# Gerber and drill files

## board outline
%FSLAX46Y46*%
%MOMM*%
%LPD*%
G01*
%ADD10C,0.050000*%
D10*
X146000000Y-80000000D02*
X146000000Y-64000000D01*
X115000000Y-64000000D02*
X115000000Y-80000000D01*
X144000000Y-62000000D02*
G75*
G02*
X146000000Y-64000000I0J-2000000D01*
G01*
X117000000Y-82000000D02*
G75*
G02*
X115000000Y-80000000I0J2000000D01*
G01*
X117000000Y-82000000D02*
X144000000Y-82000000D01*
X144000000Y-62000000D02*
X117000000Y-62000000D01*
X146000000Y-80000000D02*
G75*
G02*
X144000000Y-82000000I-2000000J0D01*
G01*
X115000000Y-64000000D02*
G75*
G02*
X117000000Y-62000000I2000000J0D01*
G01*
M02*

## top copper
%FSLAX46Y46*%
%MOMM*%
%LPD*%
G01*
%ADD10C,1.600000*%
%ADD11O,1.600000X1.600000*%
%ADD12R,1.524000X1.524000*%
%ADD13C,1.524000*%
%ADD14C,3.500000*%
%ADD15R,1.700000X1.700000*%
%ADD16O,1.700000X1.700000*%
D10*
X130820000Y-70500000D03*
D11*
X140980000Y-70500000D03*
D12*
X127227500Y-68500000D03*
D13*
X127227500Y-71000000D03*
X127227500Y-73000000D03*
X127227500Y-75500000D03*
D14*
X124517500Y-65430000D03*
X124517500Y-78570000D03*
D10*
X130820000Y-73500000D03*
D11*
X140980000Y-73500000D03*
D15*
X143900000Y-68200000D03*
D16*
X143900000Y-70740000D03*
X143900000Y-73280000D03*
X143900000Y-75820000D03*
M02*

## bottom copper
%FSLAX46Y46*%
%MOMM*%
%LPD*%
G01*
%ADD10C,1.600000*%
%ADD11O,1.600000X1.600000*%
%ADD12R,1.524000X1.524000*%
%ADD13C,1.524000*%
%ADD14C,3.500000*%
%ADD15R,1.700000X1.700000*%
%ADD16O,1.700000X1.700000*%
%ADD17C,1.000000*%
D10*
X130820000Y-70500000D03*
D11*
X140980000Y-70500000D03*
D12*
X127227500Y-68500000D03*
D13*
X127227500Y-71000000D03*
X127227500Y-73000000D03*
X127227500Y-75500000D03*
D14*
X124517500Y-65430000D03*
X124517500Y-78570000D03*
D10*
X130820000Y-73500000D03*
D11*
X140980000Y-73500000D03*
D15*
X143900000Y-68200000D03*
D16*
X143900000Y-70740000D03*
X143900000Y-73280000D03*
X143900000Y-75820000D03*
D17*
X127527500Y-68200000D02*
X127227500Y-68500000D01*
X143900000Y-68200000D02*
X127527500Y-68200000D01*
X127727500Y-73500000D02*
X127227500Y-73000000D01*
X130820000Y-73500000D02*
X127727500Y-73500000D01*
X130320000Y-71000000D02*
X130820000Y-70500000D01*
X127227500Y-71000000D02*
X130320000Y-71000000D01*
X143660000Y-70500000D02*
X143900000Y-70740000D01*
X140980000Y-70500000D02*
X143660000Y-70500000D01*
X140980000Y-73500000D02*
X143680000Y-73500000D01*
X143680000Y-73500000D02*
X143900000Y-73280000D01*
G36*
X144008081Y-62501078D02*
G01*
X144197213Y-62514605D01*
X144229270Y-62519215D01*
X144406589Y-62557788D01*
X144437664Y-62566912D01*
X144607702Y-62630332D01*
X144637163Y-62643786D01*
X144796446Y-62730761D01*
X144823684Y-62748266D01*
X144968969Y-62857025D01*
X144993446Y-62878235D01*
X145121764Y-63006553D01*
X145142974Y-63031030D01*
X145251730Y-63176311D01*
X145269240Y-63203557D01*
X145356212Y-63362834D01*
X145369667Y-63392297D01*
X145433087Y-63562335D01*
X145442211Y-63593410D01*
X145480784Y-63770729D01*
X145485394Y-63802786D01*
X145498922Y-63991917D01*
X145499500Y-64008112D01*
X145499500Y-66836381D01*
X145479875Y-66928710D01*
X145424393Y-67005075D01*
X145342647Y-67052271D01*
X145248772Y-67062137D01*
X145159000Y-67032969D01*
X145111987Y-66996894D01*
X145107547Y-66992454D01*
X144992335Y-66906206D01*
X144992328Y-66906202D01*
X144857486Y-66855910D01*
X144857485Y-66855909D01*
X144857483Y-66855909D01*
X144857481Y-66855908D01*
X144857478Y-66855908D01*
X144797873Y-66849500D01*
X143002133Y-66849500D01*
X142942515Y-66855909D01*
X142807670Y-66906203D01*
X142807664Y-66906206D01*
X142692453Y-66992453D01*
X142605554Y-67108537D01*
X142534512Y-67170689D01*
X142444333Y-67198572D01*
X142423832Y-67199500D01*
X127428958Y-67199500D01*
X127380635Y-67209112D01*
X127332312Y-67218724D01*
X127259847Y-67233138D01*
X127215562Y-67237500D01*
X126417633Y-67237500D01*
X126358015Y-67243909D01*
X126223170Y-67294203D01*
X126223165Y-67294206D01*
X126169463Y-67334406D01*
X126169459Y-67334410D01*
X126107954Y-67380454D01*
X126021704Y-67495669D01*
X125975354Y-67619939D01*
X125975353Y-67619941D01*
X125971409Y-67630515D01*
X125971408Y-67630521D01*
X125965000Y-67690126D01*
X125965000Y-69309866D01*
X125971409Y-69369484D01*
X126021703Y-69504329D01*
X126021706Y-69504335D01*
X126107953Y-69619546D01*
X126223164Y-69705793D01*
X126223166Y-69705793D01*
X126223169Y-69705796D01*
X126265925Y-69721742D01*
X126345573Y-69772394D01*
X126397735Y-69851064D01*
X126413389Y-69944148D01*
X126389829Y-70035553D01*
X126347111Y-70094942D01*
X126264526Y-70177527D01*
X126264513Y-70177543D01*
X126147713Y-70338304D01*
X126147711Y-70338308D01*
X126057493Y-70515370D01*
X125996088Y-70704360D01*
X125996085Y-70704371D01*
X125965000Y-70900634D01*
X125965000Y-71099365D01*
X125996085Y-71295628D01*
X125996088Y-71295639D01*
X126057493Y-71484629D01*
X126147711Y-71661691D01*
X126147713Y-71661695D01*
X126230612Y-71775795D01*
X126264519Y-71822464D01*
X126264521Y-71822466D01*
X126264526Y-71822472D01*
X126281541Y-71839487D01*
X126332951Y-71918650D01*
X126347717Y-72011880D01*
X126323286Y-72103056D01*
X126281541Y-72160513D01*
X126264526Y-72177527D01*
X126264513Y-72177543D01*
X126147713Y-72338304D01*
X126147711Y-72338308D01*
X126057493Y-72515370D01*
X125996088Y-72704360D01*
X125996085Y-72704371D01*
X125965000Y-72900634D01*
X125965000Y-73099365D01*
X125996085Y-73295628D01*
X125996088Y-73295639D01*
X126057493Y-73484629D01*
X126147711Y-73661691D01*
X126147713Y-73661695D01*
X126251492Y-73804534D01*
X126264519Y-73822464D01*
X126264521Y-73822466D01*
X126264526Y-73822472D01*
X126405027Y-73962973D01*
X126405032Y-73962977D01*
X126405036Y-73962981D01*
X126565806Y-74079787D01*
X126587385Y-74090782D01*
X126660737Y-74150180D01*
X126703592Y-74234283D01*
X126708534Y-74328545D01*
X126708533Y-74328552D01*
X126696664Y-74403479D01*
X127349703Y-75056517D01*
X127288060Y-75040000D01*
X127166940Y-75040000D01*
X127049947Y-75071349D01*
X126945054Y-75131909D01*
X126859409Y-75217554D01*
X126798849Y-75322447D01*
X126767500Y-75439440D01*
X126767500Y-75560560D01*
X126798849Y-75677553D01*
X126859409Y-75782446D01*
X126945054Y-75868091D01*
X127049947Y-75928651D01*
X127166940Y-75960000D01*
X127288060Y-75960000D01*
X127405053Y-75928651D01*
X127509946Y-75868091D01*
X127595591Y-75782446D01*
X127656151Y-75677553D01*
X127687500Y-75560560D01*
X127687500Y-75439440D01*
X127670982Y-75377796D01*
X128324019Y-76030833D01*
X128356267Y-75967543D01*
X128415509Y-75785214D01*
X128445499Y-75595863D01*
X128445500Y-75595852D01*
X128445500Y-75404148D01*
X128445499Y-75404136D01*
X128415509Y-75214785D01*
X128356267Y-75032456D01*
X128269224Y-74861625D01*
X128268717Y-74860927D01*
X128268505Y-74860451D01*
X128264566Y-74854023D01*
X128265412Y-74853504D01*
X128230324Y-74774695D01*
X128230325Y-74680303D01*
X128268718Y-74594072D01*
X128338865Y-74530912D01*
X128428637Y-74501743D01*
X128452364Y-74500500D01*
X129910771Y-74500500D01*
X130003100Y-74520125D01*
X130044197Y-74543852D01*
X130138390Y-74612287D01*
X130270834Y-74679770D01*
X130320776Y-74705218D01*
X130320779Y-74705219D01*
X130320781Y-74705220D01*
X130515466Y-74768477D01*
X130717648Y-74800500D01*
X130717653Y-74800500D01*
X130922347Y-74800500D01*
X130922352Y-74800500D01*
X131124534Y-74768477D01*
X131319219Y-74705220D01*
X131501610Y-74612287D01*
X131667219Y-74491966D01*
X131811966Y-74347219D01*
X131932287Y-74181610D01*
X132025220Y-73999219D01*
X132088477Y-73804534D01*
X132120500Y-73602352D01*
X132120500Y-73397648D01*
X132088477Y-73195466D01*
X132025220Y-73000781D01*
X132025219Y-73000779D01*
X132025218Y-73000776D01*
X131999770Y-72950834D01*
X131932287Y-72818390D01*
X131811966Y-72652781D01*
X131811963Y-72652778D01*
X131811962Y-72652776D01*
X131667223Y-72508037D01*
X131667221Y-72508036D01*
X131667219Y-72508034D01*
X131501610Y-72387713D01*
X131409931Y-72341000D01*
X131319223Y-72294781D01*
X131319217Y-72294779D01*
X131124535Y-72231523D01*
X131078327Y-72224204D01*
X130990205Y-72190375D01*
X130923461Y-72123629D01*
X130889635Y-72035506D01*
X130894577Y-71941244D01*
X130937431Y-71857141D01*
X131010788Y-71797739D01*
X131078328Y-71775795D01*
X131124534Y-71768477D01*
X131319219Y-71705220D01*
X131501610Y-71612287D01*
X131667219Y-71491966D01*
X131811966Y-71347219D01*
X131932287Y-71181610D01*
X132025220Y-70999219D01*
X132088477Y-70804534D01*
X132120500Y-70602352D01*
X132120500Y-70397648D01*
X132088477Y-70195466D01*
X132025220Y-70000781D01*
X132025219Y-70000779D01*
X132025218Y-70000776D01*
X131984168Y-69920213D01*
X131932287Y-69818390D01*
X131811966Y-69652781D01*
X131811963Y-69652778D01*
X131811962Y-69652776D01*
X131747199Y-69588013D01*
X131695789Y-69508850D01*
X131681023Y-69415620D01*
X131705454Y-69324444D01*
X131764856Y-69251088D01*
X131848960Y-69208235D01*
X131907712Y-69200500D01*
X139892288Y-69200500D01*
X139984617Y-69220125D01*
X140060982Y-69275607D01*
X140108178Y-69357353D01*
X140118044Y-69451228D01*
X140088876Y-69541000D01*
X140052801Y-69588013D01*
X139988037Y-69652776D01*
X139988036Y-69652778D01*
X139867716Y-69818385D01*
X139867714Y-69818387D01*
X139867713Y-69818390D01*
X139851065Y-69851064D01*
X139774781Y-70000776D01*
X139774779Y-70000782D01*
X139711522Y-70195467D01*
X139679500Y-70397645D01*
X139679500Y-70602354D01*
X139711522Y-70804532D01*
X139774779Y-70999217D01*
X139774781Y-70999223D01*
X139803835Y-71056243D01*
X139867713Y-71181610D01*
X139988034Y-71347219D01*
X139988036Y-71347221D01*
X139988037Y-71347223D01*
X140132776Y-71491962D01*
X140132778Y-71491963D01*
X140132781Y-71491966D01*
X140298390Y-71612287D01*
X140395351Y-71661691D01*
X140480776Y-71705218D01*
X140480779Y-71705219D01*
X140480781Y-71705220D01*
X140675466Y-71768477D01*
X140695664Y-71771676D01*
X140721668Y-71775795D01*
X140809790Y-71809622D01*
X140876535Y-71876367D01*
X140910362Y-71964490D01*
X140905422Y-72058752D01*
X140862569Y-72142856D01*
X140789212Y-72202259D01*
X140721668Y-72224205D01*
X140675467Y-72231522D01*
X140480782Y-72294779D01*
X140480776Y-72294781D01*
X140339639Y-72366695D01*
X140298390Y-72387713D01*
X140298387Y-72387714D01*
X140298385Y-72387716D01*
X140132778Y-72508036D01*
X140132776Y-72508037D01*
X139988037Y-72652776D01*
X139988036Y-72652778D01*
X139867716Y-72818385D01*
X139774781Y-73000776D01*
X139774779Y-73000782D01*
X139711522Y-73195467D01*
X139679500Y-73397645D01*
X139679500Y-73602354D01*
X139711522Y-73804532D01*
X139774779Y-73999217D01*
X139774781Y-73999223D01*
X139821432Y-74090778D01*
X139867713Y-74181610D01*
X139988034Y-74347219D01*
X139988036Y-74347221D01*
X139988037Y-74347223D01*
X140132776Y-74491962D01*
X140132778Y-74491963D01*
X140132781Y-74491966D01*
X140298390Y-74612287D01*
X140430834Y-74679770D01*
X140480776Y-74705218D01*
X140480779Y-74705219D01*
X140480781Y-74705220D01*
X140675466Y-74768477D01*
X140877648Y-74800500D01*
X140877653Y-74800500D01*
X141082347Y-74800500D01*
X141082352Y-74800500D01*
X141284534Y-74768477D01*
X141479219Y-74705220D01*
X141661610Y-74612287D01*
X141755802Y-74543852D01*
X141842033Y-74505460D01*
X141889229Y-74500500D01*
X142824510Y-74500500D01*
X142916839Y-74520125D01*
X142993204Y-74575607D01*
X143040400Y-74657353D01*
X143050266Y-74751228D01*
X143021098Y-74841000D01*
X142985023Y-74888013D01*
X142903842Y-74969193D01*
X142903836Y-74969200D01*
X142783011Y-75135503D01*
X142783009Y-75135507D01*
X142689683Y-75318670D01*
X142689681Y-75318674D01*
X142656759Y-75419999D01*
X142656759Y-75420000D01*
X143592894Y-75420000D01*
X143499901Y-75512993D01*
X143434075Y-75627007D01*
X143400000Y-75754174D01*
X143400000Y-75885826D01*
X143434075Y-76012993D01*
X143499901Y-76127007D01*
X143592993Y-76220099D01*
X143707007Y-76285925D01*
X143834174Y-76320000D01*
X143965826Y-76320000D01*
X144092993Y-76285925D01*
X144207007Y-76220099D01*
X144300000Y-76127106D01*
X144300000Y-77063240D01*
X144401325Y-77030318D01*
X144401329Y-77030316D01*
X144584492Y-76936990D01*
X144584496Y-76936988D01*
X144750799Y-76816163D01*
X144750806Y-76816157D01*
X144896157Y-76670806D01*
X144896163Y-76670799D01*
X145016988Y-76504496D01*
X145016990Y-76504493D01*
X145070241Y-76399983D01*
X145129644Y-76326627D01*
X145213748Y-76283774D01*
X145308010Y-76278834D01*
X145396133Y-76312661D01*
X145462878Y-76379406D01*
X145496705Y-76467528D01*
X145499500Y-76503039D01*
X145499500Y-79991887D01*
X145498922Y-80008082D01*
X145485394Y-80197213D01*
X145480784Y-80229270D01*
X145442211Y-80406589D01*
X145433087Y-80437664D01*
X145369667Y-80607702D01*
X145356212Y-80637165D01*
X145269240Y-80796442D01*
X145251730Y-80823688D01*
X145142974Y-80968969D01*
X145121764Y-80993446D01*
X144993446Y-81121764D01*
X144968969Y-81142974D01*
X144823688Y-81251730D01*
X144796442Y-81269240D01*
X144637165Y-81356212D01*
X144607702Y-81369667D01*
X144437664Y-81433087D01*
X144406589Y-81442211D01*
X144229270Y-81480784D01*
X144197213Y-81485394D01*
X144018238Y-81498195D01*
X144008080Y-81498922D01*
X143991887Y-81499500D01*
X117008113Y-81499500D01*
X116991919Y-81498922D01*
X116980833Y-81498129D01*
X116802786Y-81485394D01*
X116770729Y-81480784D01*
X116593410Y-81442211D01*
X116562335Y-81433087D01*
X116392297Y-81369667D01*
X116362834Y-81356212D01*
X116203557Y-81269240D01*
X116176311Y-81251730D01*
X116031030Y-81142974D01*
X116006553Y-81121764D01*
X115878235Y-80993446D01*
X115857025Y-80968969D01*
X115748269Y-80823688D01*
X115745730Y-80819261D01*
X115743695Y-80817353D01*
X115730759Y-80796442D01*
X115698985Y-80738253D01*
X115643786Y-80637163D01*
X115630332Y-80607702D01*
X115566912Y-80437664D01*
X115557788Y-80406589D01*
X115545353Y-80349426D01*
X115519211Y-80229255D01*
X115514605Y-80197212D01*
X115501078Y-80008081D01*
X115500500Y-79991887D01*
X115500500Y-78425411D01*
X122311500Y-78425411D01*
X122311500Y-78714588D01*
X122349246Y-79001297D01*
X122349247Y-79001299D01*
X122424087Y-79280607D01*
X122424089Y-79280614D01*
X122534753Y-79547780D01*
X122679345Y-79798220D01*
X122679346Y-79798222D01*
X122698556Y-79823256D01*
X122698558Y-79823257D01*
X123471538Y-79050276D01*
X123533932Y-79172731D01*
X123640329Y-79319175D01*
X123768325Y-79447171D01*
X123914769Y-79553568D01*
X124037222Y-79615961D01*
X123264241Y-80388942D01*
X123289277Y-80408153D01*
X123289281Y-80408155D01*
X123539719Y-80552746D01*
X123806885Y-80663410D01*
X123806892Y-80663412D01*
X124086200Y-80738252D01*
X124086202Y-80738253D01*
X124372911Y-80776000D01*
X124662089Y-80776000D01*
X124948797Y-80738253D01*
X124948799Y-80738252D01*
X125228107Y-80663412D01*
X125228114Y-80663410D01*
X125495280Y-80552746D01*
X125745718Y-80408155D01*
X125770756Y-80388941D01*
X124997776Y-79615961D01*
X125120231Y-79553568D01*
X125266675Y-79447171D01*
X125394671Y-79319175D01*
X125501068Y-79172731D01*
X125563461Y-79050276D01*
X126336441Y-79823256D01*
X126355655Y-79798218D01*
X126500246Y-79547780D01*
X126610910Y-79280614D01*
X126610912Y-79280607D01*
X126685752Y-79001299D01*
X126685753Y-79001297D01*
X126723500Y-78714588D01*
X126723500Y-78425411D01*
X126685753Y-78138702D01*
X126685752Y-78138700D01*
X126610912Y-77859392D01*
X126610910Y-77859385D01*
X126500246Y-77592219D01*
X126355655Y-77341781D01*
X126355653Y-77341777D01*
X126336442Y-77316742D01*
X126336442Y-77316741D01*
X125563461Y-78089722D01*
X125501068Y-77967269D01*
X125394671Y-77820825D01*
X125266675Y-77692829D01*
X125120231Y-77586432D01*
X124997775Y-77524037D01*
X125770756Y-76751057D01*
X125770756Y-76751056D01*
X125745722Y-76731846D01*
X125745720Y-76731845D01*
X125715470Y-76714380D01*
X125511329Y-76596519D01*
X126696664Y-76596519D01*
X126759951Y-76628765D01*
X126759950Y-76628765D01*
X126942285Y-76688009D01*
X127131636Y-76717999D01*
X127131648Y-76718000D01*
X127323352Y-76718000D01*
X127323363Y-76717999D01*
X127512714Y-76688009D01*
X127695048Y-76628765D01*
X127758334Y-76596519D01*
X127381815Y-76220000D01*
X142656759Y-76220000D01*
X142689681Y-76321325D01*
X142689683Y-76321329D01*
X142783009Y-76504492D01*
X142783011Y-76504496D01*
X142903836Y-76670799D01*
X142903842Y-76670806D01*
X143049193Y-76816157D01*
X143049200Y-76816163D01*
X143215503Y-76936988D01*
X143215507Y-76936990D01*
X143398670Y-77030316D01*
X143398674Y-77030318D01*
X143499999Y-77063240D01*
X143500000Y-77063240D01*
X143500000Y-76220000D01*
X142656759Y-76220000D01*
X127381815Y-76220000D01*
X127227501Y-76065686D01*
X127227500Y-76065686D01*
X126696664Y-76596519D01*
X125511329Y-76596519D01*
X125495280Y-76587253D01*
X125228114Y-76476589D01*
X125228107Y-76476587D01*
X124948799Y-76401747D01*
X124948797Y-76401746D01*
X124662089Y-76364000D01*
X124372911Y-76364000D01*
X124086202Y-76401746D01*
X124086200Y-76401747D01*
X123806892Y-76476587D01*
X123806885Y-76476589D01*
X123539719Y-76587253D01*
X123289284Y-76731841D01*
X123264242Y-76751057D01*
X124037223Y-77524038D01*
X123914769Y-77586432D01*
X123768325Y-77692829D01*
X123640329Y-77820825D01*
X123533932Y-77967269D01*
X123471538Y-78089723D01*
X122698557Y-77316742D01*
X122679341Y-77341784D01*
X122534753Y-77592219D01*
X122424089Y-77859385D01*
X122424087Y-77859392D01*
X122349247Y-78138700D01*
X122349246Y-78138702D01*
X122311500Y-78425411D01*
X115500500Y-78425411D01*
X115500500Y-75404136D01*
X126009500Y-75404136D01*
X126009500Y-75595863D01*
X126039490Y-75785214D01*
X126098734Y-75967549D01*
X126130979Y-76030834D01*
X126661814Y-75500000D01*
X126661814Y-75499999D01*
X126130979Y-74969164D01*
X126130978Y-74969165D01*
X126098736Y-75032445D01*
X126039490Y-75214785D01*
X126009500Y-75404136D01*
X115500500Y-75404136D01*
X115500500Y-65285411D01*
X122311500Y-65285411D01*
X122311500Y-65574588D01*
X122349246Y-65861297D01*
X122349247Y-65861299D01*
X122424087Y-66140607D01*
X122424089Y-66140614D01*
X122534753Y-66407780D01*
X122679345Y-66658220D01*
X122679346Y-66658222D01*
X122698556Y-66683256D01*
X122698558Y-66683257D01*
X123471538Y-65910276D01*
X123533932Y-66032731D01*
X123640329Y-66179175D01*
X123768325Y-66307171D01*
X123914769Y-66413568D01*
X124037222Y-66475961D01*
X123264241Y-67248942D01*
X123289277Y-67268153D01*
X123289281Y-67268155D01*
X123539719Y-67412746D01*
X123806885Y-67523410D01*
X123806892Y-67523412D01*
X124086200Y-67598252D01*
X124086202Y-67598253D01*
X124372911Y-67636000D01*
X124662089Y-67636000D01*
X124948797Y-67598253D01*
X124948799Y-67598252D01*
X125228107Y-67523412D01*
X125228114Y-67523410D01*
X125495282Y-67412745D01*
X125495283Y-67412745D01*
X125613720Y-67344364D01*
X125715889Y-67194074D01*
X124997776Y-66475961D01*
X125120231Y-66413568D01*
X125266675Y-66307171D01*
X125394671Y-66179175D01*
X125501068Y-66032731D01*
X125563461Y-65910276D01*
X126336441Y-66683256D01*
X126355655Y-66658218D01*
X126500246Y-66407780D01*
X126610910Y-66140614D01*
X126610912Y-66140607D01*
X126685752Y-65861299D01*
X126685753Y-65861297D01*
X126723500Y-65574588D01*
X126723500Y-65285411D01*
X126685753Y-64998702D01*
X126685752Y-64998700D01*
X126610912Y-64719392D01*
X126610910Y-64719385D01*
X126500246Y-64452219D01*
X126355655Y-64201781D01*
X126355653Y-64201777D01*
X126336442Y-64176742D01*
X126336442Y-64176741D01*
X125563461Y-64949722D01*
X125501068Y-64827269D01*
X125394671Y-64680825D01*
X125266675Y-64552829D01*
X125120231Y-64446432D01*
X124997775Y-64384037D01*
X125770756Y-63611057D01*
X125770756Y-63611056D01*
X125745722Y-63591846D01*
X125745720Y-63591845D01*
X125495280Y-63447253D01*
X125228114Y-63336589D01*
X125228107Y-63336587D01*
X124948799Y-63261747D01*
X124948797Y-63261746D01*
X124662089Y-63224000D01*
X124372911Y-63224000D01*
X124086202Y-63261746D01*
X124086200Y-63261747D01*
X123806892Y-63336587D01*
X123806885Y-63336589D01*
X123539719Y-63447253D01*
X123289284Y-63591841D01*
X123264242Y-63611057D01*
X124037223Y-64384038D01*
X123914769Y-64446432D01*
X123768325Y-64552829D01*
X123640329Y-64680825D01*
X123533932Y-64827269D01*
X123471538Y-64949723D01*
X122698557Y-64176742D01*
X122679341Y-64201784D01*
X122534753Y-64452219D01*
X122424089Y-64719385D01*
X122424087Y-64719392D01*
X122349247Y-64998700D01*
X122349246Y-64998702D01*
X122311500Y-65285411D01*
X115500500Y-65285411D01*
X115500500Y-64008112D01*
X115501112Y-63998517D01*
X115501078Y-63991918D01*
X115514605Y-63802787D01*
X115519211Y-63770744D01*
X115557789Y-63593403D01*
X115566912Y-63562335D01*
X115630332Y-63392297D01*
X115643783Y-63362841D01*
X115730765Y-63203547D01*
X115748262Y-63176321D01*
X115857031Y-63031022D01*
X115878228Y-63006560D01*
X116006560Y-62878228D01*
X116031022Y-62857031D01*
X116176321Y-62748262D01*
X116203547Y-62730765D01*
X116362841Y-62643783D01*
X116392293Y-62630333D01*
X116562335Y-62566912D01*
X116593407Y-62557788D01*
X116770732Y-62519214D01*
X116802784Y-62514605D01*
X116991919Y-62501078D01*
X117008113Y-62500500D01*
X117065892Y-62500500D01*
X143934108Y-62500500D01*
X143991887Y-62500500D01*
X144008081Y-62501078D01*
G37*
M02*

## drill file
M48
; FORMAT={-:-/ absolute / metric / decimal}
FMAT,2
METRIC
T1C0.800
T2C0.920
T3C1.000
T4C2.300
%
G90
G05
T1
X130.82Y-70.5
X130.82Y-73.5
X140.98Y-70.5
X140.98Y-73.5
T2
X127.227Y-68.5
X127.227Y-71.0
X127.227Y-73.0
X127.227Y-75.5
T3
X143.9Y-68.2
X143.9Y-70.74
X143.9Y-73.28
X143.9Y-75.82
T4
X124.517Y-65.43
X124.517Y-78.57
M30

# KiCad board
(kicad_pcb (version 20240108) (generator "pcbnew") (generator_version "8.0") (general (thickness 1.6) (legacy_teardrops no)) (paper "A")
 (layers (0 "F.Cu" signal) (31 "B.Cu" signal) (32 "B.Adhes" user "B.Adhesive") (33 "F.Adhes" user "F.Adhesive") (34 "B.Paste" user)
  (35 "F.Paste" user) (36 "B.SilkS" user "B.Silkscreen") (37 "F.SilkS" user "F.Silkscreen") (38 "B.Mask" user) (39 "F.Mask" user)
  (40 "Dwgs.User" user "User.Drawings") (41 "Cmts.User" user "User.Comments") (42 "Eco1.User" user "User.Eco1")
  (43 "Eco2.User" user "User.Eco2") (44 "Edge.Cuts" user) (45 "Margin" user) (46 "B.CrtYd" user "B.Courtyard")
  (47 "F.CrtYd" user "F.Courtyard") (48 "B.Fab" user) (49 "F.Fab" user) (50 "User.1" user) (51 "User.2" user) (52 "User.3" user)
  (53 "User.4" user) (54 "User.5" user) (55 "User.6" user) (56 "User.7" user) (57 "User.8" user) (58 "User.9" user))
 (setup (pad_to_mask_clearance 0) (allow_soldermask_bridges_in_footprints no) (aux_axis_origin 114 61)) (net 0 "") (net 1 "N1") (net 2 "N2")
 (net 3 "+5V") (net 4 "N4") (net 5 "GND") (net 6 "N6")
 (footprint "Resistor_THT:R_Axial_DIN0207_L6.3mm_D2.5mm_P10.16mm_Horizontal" (layer "F.Cu") (at 130.82 70.5)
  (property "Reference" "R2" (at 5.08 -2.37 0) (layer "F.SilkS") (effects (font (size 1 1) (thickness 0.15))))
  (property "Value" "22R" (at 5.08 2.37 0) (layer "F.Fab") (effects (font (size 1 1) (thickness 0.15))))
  (pad "1" thru_hole circle (at 0 0) (size 1.6 1.6) (drill 0.8) (layers "*.Cu" "*.Mask") (remove_unused_layers no) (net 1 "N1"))
  (pad "2" thru_hole oval (at 10.16 0) (size 1.6 1.6) (drill 0.8) (layers "*.Cu" "*.Mask") (remove_unused_layers no) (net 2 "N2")))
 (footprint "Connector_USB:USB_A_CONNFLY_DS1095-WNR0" (layer "F.Cu") (at 127.2275 68.5 -90)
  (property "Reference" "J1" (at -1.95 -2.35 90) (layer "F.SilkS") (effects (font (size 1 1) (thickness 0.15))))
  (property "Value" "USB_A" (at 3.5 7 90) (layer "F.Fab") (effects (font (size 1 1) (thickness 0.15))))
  (pad "1" thru_hole rect (at 0 0 270) (size 1.524 1.524) (drill 0.92) (layers "*.Cu" "*.Mask") (remove_unused_layers no) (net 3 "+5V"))
  (pad "2" thru_hole circle (at 2.5 0 270) (size 1.524 1.524) (drill 0.92) (layers "*.Cu" "*.Mask") (remove_unused_layers no) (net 1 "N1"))
  (pad "3" thru_hole circle (at 4.5 0 270) (size 1.524 1.524) (drill 0.92) (layers "*.Cu" "*.Mask") (remove_unused_layers no) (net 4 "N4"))
  (pad "4" thru_hole circle (at 7 0 270) (size 1.524 1.524) (drill 0.92) (layers "*.Cu" "*.Mask") (remove_unused_layers no) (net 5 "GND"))
  (pad "5" thru_hole circle (at -3.07 2.71 270) (size 3.5 3.5) (drill 2.3) (layers "*.Cu" "*.Mask") (remove_unused_layers no) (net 5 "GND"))
  (pad "5" thru_hole circle (at 10.07 2.71 270) (size 3.5 3.5) (drill 2.3) (layers "*.Cu" "*.Mask") (remove_unused_layers no) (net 5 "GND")))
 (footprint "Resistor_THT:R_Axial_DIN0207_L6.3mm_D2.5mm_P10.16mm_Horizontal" (layer "F.Cu") (at 130.82 73.5)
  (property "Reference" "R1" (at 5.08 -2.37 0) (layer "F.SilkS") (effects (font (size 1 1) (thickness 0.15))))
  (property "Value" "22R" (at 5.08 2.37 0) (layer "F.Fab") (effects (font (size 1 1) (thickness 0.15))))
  (pad "1" thru_hole circle (at 0 0) (size 1.6 1.6) (drill 0.8) (layers "*.Cu" "*.Mask") (remove_unused_layers no) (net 4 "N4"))
  (pad "2" thru_hole oval (at 10.16 0) (size 1.6 1.6) (drill 0.8) (layers "*.Cu" "*.Mask") (remove_unused_layers no) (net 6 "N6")))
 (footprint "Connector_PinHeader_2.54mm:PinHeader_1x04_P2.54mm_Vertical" (layer "B.Cu") (at 143.9 68.2 180)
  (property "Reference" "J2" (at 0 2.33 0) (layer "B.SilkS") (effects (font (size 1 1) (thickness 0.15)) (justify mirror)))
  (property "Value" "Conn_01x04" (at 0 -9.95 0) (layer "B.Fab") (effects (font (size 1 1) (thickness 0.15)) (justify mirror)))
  (pad "1" thru_hole rect (at 0 0 180) (size 1.7 1.7) (drill 1) (layers "*.Cu" "*.Mask") (remove_unused_layers no) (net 3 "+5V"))
  (pad "2" thru_hole oval (at 0 -2.54 180) (size 1.7 1.7) (drill 1) (layers "*.Cu" "*.Mask") (remove_unused_layers no) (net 2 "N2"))
  (pad "3" thru_hole oval (at 0 -5.08 180) (size 1.7 1.7) (drill 1) (layers "*.Cu" "*.Mask") (remove_unused_layers no) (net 6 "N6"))
  (pad "4" thru_hole oval (at 0 -7.62 180) (size 1.7 1.7) (drill 1) (layers "*.Cu" "*.Mask") (remove_unused_layers no) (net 5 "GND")))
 (gr_line (start 146 80) (end 146 64) (stroke (width 0.05) (type default)) (layer "Edge.Cuts"))
 (gr_line (start 115 64) (end 115 80) (stroke (width 0.05) (type default)) (layer "Edge.Cuts"))
 (gr_arc (start 144 62) (mid 145.414214 62.585786) (end 146 64) (stroke (width 0.05) (type default)) (layer "Edge.Cuts"))
 (gr_arc (start 117 82) (mid 115.585786 81.414214) (end 115 80) (stroke (width 0.05) (type default)) (layer "Edge.Cuts"))
 (gr_line (start 117 82) (end 144 82) (stroke (width 0.05) (type default)) (layer "Edge.Cuts"))
 (gr_line (start 144 62) (end 117 62) (stroke (width 0.05) (type default)) (layer "Edge.Cuts"))
 (gr_arc (start 146 80) (mid 145.414214 81.414214) (end 144 82) (stroke (width 0.05) (type default)) (layer "Edge.Cuts"))
 (gr_arc (start 115 64) (mid 115.585786 62.585786) (end 117 62) (stroke (width 0.05) (type default)) (layer "Edge.Cuts"))
 (segment (start 127.5275 68.2) (end 127.2275 68.5) (width 1) (layer "B.Cu") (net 3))
 (segment (start 143.9 68.2) (end 127.5275 68.2) (width 1) (layer "B.Cu") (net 3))
 (segment (start 127.7275 73.5) (end 127.2275 73) (width 1) (layer "B.Cu") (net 4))
 (segment (start 130.82 73.5) (end 127.7275 73.5) (width 1) (layer "B.Cu") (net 4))
 (segment (start 130.32 71) (end 130.82 70.5) (width 1) (layer "B.Cu") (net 1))
 (segment (start 127.2275 71) (end 130.32 71) (width 1) (layer "B.Cu") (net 1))
 (segment (start 143.66 70.5) (end 143.9 70.74) (width 1) (layer "B.Cu") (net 2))
 (segment (start 140.98 70.5) (end 143.66 70.5) (width 1) (layer "B.Cu") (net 2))
 (segment (start 140.98 73.5) (end 143.68 73.5) (width 1) (layer "B.Cu") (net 6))
 (segment (start 143.68 73.5) (end 143.9 73.28) (width 1) (layer "B.Cu") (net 6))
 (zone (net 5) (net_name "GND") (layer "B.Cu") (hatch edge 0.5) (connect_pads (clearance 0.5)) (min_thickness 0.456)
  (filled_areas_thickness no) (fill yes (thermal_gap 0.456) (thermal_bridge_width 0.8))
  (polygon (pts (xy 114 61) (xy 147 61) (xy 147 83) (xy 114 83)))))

